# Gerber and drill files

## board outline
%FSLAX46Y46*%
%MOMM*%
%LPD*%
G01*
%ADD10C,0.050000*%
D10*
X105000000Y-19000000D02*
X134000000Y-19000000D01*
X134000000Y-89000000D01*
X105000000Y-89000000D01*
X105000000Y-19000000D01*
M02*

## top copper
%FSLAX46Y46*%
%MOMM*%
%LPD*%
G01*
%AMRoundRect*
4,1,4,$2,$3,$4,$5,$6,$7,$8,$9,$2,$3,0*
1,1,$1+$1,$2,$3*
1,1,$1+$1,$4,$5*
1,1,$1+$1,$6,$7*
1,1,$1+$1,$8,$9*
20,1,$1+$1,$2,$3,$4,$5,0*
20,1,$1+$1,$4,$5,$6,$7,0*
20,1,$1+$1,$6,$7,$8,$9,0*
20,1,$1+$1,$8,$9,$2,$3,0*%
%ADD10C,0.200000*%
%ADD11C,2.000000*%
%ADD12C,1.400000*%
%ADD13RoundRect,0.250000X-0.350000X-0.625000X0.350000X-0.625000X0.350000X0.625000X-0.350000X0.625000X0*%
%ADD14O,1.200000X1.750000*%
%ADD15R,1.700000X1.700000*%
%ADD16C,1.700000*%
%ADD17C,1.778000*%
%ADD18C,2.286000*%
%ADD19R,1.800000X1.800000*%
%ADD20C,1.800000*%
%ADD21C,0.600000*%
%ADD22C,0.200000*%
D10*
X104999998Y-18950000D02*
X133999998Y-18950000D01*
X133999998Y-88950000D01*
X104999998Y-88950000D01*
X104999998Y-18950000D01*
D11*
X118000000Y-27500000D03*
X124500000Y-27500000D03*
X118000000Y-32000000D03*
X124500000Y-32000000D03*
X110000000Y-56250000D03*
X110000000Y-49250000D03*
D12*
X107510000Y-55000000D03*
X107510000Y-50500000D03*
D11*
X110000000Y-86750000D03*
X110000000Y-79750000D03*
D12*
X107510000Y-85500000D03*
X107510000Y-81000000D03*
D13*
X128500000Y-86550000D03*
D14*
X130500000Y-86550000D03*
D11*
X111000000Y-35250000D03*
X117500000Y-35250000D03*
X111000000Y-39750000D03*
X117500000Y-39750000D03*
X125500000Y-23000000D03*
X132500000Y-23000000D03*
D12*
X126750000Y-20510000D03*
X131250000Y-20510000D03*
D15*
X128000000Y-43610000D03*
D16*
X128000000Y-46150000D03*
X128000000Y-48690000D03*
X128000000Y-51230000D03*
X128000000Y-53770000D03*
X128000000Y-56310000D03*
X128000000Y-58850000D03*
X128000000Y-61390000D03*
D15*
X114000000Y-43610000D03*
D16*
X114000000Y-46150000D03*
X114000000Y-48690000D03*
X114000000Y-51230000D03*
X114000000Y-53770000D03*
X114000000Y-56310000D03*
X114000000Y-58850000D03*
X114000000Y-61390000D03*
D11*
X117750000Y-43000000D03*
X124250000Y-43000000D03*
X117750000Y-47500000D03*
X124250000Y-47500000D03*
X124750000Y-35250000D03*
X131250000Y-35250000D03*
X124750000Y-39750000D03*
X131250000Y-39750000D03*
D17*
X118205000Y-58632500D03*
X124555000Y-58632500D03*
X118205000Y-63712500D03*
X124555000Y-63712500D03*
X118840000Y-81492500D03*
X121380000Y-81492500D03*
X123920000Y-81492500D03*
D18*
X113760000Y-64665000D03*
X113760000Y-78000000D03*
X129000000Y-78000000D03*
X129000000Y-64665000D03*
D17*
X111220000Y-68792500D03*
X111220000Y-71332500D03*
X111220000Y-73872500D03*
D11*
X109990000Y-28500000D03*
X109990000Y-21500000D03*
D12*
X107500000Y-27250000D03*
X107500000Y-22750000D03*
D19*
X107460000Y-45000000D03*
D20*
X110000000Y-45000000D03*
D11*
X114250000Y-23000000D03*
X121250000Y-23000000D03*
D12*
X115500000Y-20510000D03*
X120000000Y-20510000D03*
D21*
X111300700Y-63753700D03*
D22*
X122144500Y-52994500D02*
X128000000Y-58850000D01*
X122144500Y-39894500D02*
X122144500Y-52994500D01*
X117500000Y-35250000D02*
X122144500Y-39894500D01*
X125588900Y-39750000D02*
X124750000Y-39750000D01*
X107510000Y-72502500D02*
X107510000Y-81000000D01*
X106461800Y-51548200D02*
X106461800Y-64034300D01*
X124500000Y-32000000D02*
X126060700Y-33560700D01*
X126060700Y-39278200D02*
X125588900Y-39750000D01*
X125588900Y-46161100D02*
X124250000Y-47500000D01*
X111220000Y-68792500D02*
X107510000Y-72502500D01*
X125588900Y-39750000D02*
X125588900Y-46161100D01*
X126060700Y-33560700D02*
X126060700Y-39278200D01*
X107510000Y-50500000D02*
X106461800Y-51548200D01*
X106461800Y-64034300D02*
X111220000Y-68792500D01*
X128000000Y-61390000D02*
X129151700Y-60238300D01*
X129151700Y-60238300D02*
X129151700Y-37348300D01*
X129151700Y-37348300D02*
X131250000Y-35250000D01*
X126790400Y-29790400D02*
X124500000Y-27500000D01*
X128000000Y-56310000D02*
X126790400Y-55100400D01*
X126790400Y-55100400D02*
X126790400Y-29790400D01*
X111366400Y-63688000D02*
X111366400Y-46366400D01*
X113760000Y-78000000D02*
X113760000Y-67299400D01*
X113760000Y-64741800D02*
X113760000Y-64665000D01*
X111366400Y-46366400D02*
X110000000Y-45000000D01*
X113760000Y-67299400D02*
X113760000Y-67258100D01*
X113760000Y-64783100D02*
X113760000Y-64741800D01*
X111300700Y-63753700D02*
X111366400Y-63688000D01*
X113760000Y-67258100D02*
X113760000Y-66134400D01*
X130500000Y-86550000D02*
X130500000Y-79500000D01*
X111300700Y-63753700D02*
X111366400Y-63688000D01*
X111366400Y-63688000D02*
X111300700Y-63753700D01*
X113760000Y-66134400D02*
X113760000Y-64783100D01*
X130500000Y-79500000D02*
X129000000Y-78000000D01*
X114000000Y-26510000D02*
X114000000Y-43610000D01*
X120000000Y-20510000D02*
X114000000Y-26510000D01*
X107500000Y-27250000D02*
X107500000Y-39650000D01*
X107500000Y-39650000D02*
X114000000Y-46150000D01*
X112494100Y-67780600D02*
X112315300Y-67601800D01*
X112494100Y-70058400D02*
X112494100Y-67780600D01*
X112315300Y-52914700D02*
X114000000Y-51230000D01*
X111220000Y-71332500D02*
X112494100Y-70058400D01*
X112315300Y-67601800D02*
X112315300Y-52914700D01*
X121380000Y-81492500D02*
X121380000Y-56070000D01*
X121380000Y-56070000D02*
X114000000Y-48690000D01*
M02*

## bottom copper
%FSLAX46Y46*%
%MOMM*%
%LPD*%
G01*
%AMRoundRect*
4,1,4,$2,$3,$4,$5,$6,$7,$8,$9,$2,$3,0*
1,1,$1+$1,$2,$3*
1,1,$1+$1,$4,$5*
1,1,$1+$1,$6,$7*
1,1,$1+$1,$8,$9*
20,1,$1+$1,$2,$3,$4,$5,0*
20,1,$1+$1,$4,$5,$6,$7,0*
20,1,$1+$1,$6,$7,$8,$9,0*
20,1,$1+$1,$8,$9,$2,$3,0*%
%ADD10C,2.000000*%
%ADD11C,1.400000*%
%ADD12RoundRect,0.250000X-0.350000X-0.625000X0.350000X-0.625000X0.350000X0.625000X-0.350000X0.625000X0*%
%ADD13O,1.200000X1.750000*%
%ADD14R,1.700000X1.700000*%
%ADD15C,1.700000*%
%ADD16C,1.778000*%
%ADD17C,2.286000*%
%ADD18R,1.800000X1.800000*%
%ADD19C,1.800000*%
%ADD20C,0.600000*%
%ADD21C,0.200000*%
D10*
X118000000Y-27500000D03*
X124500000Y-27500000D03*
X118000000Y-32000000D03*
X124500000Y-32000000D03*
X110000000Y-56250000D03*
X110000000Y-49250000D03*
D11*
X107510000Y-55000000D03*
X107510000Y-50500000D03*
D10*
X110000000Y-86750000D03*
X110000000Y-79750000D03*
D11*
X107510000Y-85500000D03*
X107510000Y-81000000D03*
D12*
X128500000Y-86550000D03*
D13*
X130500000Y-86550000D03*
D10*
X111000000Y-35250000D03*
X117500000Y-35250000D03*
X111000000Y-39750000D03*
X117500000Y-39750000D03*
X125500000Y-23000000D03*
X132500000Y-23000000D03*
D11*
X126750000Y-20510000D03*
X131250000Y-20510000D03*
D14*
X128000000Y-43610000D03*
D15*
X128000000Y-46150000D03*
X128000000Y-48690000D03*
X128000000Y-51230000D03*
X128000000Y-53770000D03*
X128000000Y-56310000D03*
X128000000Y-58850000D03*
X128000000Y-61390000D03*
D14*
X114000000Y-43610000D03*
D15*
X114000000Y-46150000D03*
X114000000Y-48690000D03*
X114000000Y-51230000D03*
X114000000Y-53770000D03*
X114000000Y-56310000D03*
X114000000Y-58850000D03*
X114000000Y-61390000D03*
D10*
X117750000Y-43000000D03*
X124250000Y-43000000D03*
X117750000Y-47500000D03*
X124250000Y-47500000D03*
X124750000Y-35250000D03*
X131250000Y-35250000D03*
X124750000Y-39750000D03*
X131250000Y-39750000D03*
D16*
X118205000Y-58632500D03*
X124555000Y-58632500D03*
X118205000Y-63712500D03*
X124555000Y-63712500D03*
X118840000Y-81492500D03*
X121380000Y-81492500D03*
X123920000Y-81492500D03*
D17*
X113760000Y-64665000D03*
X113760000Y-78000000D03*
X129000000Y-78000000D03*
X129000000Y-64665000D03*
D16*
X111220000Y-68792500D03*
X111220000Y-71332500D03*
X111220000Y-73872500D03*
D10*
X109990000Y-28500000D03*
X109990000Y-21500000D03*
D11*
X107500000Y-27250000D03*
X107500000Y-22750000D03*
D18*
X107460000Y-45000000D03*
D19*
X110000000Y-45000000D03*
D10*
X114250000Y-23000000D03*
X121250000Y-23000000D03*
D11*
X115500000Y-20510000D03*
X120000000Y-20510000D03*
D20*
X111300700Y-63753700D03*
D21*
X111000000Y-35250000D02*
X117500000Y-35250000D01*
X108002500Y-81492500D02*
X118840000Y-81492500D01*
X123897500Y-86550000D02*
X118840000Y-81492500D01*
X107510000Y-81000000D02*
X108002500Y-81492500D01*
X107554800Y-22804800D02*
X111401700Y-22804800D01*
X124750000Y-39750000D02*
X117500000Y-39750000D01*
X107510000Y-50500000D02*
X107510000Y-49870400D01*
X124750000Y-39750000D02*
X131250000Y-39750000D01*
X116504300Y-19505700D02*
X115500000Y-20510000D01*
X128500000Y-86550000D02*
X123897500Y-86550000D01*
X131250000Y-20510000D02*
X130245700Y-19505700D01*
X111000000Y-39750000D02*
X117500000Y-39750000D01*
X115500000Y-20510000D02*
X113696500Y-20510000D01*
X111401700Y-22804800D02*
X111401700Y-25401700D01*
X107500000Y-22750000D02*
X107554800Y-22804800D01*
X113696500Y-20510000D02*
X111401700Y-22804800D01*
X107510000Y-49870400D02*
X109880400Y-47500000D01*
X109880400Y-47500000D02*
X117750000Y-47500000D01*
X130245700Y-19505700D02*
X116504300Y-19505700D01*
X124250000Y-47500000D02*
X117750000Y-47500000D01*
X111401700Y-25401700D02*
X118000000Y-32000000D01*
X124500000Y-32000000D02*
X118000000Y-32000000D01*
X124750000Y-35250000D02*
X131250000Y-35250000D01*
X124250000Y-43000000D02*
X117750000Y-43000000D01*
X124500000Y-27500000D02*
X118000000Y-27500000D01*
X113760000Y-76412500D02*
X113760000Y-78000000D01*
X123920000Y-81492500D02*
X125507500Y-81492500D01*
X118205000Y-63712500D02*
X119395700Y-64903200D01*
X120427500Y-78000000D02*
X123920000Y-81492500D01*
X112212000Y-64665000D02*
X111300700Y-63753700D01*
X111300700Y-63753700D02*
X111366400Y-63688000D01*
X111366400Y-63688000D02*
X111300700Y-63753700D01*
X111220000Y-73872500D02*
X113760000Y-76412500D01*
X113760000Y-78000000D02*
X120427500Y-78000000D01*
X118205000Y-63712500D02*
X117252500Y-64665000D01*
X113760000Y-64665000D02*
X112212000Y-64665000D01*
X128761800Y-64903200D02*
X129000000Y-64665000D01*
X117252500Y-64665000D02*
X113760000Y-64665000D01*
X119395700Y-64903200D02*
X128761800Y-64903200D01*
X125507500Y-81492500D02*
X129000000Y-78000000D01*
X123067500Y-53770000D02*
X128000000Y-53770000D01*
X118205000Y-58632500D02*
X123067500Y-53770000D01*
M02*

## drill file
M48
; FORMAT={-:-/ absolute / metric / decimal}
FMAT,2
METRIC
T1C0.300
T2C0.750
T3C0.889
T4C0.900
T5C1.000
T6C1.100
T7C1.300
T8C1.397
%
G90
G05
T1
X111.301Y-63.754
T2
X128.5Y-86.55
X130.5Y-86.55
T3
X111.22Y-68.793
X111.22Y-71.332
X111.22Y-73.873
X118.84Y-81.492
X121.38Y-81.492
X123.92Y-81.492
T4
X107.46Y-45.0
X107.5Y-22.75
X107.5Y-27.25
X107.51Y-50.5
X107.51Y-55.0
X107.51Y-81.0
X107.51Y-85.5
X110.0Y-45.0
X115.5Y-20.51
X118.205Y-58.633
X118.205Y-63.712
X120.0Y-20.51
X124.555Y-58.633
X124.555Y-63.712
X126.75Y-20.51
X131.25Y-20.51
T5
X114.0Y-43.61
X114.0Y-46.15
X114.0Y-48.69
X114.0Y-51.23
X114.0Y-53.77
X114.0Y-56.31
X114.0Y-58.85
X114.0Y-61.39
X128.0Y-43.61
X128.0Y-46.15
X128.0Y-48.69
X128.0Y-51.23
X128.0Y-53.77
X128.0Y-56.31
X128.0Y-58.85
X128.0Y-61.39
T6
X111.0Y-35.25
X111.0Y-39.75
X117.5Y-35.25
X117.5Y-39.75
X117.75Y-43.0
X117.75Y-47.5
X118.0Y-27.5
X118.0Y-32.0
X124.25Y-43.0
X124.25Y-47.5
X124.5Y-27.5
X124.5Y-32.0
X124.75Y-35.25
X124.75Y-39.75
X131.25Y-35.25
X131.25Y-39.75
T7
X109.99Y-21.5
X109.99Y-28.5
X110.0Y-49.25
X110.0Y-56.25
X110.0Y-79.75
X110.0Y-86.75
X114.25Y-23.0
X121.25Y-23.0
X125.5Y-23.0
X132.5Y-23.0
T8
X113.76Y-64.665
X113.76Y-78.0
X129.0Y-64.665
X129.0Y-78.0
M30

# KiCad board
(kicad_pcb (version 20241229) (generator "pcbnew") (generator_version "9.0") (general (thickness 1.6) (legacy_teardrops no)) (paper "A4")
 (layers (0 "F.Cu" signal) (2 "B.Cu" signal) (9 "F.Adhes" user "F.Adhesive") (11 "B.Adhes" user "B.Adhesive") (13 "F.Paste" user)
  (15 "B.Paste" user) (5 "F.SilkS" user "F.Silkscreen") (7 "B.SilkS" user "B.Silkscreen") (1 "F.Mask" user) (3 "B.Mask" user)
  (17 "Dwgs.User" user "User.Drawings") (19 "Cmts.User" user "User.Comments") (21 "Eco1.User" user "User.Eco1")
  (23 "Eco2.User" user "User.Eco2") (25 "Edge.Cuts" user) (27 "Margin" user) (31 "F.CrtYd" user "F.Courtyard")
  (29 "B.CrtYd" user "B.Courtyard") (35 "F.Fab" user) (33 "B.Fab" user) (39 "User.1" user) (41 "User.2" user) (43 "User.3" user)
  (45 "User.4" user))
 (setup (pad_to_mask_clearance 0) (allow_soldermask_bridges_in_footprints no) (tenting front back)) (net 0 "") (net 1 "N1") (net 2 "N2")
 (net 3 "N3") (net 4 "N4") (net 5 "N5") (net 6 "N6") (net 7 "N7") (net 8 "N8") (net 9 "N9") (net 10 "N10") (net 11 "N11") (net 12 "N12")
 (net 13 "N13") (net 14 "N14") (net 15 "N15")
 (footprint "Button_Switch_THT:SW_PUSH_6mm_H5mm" (layer "F.Cu") (at 118 27.5)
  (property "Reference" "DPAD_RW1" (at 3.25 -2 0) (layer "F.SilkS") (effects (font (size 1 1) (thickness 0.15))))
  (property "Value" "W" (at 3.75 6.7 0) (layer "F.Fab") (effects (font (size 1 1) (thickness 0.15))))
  (pad "1" thru_hole circle (at 0 0 90) (size 2 2) (drill 1.1) (layers "*.Cu" "*.Mask") (remove_unused_layers no) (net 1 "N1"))
  (pad "1" thru_hole circle (at 6.5 0 90) (size 2 2) (drill 1.1) (layers "*.Cu" "*.Mask") (remove_unused_layers no) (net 1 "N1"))
  (pad "2" thru_hole circle (at 0 4.5 90) (size 2 2) (drill 1.1) (layers "*.Cu" "*.Mask") (remove_unused_layers no) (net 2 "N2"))
  (pad "2" thru_hole circle (at 6.5 4.5 90) (size 2 2) (drill 1.1) (layers "*.Cu" "*.Mask") (remove_unused_layers no) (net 2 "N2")))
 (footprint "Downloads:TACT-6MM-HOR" (layer "F.Cu") (at 107.51 52.75 90)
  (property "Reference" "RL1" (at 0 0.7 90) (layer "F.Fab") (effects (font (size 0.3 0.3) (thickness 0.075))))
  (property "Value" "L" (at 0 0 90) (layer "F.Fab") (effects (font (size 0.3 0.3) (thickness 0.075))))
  (pad "" thru_hole circle (at -3.5 2.49 90) (size 2 2) (drill 1.3) (layers "*.Cu" "*.Mask" "F.SilkS") (remove_unused_layers no))
  (pad "" thru_hole circle (at 3.5 2.49 90) (size 2 2) (drill 1.3) (layers "*.Cu" "*.Mask" "F.SilkS") (remove_unused_layers no))
  (pad "1" thru_hole circle (at -2.25 0 90) (size 1.4 1.4) (drill 0.9) (layers "*.Cu" "*.Mask" "F.SilkS") (remove_unused_layers no)
   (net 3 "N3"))
  (pad "2" thru_hole circle (at 2.25 0 90) (size 1.4 1.4) (drill 0.9) (layers "*.Cu" "*.Mask" "F.SilkS") (remove_unused_layers no)
   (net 2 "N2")))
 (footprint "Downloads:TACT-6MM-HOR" (layer "F.Cu") (at 107.51 83.25 90)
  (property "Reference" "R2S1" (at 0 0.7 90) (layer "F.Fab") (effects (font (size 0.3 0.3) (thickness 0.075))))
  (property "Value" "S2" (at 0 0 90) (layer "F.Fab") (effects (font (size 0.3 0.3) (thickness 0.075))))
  (pad "" thru_hole circle (at -3.5 2.49 90) (size 2 2) (drill 1.3) (layers "*.Cu" "*.Mask" "F.SilkS") (remove_unused_layers no))
  (pad "" thru_hole circle (at 3.5 2.49 90) (size 2 2) (drill 1.3) (layers "*.Cu" "*.Mask" "F.SilkS") (remove_unused_layers no))
  (pad "1" thru_hole circle (at -2.25 0 90) (size 1.4 1.4) (drill 0.9) (layers "*.Cu" "*.Mask" "F.SilkS") (remove_unused_layers no)
   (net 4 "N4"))
  (pad "2" thru_hole circle (at 2.25 0 90) (size 1.4 1.4) (drill 0.9) (layers "*.Cu" "*.Mask" "F.SilkS") (remove_unused_layers no)
   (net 2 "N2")))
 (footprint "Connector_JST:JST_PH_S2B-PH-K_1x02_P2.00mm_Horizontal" (layer "F.Cu") (at 128.5 86.55)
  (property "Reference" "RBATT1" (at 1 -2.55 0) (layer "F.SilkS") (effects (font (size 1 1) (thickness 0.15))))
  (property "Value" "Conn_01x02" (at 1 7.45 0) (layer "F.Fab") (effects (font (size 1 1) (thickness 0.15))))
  (pad "1" thru_hole roundrect (at 0 0) (size 1.2 1.75) (drill 0.75) (layers "*.Cu" "*.Mask") (remove_unused_layers no)
   (roundrect_rratio 0.208333) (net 2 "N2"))
  (pad "2" thru_hole oval (at 2 0) (size 1.2 1.75) (drill 0.75) (layers "*.Cu" "*.Mask") (remove_unused_layers no) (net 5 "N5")))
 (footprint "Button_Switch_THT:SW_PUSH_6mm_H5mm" (layer "F.Cu") (at 111 35.25)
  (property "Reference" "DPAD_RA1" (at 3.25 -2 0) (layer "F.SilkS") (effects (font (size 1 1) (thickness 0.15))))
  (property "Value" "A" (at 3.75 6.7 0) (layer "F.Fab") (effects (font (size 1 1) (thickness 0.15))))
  (pad "1" thru_hole circle (at 0 0 90) (size 2 2) (drill 1.1) (layers "*.Cu" "*.Mask") (remove_unused_layers no) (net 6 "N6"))
  (pad "1" thru_hole circle (at 6.5 0 90) (size 2 2) (drill 1.1) (layers "*.Cu" "*.Mask") (remove_unused_layers no) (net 6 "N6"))
  (pad "2" thru_hole circle (at 0 4.5 90) (size 2 2) (drill 1.1) (layers "*.Cu" "*.Mask") (remove_unused_layers no) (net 2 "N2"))
  (pad "2" thru_hole circle (at 6.5 4.5 90) (size 2 2) (drill 1.1) (layers "*.Cu" "*.Mask") (remove_unused_layers no) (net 2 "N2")))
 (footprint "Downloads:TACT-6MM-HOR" (layer "F.Cu") (at 129 20.51)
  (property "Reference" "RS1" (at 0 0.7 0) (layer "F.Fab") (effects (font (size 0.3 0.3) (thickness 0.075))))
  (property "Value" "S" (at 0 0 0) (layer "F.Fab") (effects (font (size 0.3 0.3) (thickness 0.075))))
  (pad "" thru_hole circle (at -3.5 2.49) (size 2 2) (drill 1.3) (layers "*.Cu" "*.Mask" "F.SilkS") (remove_unused_layers no))
  (pad "" thru_hole circle (at 3.5 2.49) (size 2 2) (drill 1.3) (layers "*.Cu" "*.Mask" "F.SilkS") (remove_unused_layers no))
  (pad "1" thru_hole circle (at -2.25 0) (size 1.4 1.4) (drill 0.9) (layers "*.Cu" "*.Mask" "F.SilkS") (remove_unused_layers no)
   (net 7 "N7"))
  (pad "2" thru_hole circle (at 2.25 0) (size 1.4 1.4) (drill 0.9) (layers "*.Cu" "*.Mask" "F.SilkS") (remove_unused_layers no) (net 2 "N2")))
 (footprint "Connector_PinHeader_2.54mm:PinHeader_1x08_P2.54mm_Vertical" (layer "F.Cu") (at 128 43.61)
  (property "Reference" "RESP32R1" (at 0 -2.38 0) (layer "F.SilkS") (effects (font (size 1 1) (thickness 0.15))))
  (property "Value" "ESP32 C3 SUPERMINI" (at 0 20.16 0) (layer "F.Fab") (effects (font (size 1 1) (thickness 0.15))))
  (pad "1" thru_hole rect (at 0 0) (size 1.7 1.7) (drill 1) (layers "*.Cu" "*.Mask") (remove_unused_layers no))
  (pad "2" thru_hole circle (at 0 2.54) (size 1.7 1.7) (drill 1) (layers "*.Cu" "*.Mask") (remove_unused_layers no))
  (pad "3" thru_hole circle (at 0 5.08) (size 1.7 1.7) (drill 1) (layers "*.Cu" "*.Mask") (remove_unused_layers no))
  (pad "4" thru_hole circle (at 0 7.62) (size 1.7 1.7) (drill 1) (layers "*.Cu" "*.Mask") (remove_unused_layers no))
  (pad "5" thru_hole circle (at 0 10.16) (size 1.7 1.7) (drill 1) (layers "*.Cu" "*.Mask") (remove_unused_layers no) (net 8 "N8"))
  (pad "6" thru_hole circle (at 0 12.7) (size 1.7 1.7) (drill 1) (layers "*.Cu" "*.Mask") (remove_unused_layers no) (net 1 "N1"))
  (pad "7" thru_hole circle (at 0 15.24) (size 1.7 1.7) (drill 1) (layers "*.Cu" "*.Mask") (remove_unused_layers no) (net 6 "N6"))
  (pad "8" thru_hole circle (at 0 17.78) (size 1.7 1.7) (drill 1) (layers "*.Cu" "*.Mask") (remove_unused_layers no) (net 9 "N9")))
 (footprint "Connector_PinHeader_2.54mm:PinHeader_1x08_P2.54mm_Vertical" (layer "F.Cu") (at 114 43.61)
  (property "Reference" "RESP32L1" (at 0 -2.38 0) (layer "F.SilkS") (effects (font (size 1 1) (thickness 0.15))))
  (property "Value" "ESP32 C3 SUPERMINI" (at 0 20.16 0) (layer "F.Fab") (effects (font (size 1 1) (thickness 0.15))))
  (pad "1" thru_hole rect (at 0 0) (size 1.7 1.7) (drill 1) (layers "*.Cu" "*.Mask") (remove_unused_layers no) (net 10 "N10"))
  (pad "2" thru_hole circle (at 0 2.54) (size 1.7 1.7) (drill 1) (layers "*.Cu" "*.Mask") (remove_unused_layers no) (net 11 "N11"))
  (pad "3" thru_hole circle (at 0 5.08) (size 1.7 1.7) (drill 1) (layers "*.Cu" "*.Mask") (remove_unused_layers no) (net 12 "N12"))
  (pad "4" thru_hole circle (at 0 7.62) (size 1.7 1.7) (drill 1) (layers "*.Cu" "*.Mask") (remove_unused_layers no) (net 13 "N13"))
  (pad "5" thru_hole circle (at 0 10.16) (size 1.7 1.7) (drill 1) (layers "*.Cu" "*.Mask") (remove_unused_layers no))
  (pad "6" thru_hole circle (at 0 12.7) (size 1.7 1.7) (drill 1) (layers "*.Cu" "*.Mask") (remove_unused_layers no))
  (pad "7" thru_hole circle (at 0 15.24) (size 1.7 1.7) (drill 1) (layers "*.Cu" "*.Mask") (remove_unused_layers no))
  (pad "8" thru_hole circle (at 0 17.78) (size 1.7 1.7) (drill 1) (layers "*.Cu" "*.Mask") (remove_unused_layers no)))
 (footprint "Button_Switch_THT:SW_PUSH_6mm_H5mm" (layer "F.Cu") (at 117.75 43)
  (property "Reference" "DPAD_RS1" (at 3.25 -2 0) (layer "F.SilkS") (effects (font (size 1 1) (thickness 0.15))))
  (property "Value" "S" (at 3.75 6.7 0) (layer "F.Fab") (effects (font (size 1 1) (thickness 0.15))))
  (pad "1" thru_hole circle (at 0 0 90) (size 2 2) (drill 1.1) (layers "*.Cu" "*.Mask") (remove_unused_layers no) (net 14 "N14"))
  (pad "1" thru_hole circle (at 6.5 0 90) (size 2 2) (drill 1.1) (layers "*.Cu" "*.Mask") (remove_unused_layers no) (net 14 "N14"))
  (pad "2" thru_hole circle (at 0 4.5 90) (size 2 2) (drill 1.1) (layers "*.Cu" "*.Mask") (remove_unused_layers no) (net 2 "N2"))
  (pad "2" thru_hole circle (at 6.5 4.5 90) (size 2 2) (drill 1.1) (layers "*.Cu" "*.Mask") (remove_unused_layers no) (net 2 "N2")))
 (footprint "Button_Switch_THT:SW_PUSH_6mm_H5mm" (layer "F.Cu") (at 124.75 35.25)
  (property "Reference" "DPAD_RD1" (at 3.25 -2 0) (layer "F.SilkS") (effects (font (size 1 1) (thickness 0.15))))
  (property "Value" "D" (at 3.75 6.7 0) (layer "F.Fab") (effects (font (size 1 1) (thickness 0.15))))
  (pad "1" thru_hole circle (at 0 0 90) (size 2 2) (drill 1.1) (layers "*.Cu" "*.Mask") (remove_unused_layers no) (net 9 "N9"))
  (pad "1" thru_hole circle (at 6.5 0 90) (size 2 2) (drill 1.1) (layers "*.Cu" "*.Mask") (remove_unused_layers no) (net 9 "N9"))
  (pad "2" thru_hole circle (at 0 4.5 90) (size 2 2) (drill 1.1) (layers "*.Cu" "*.Mask") (remove_unused_layers no) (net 2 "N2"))
  (pad "2" thru_hole circle (at 6.5 4.5 90) (size 2 2) (drill 1.1) (layers "*.Cu" "*.Mask") (remove_unused_layers no) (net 2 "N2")))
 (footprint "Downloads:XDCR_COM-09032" (layer "F.Cu") (at 121.38 71.3325)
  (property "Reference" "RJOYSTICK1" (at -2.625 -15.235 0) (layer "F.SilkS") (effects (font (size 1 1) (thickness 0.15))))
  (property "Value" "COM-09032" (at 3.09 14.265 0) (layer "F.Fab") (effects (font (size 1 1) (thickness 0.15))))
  (pad "B1A" thru_hole circle (at -3.175 -12.7) (size 1.778 1.778) (drill 0.9) (layers "*.Cu" "*.Mask") (remove_unused_layers no)
   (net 8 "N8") (solder_mask_margin 0.102))
  (pad "B1B" thru_hole circle (at 3.175 -12.7) (size 1.778 1.778) (drill 0.9) (layers "*.Cu" "*.Mask") (remove_unused_layers no)
   (solder_mask_margin 0.102))
  (pad "B2A" thru_hole circle (at -3.175 -7.62) (size 1.778 1.778) (drill 0.9) (layers "*.Cu" "*.Mask") (remove_unused_layers no)
   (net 5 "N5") (solder_mask_margin 0.102))
  (pad "B2B" thru_hole circle (at 3.175 -7.62) (size 1.778 1.778) (drill 0.9) (layers "*.Cu" "*.Mask") (remove_unused_layers no)
   (solder_mask_margin 0.102))
  (pad "H1" thru_hole circle (at -2.54 10.16) (size 1.778 1.778) (drill 0.889) (layers "*.Cu" "*.Mask") (remove_unused_layers no)
   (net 2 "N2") (solder_mask_margin 0.102))
  (pad "H2" thru_hole circle (at 0 10.16) (size 1.778 1.778) (drill 0.889) (layers "*.Cu" "*.Mask") (remove_unused_layers no) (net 12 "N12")
   (solder_mask_margin 0.102))
  (pad "H3" thru_hole circle (at 2.54 10.16) (size 1.778 1.778) (drill 0.889) (layers "*.Cu" "*.Mask") (remove_unused_layers no)
   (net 5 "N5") (solder_mask_margin 0.102))
  (pad "S1" thru_hole circle (at -7.62 -6.6675) (size 2.286 2.286) (drill 1.397) (layers "*.Cu" "*.Mask") (remove_unused_layers no)
   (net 5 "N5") (solder_mask_margin 0.102))
  (pad "S2" thru_hole circle (at -7.62 6.6675) (size 2.286 2.286) (drill 1.397) (layers "*.Cu" "*.Mask") (remove_unused_layers no)
   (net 5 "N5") (solder_mask_margin 0.102))
  (pad "S3" thru_hole circle (at 7.62 6.6675) (size 2.286 2.286) (drill 1.397) (layers "*.Cu" "*.Mask") (remove_unused_layers no)
   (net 5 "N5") (solder_mask_margin 0.102))
  (pad "S4" thru_hole circle (at 7.62 -6.6675) (size 2.286 2.286) (drill 1.397) (layers "*.Cu" "*.Mask") (remove_unused_layers no)
   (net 5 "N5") (solder_mask_margin 0.102))
  (pad "V1" thru_hole circle (at -10.16 -2.54) (size 1.778 1.778) (drill 0.889) (layers "*.Cu" "*.Mask") (remove_unused_layers no)
   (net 2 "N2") (solder_mask_margin 0.102))
  (pad "V2" thru_hole circle (at -10.16 0) (size 1.778 1.778) (drill 0.889) (layers "*.Cu" "*.Mask") (remove_unused_layers no)
   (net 13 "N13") (solder_mask_margin 0.102))
  (pad "V3" thru_hole circle (at -10.16 2.54) (size 1.778 1.778) (drill 0.889) (layers "*.Cu" "*.Mask") (remove_unused_layers no)
   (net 5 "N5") (solder_mask_margin 0.102)))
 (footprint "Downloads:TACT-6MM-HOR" (layer "F.Cu") (at 107.5 25 90)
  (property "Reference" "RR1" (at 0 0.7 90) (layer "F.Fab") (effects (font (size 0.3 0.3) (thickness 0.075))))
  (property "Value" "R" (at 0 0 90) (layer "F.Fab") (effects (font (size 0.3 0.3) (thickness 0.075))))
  (pad "" thru_hole circle (at -3.5 2.49 90) (size 2 2) (drill 1.3) (layers "*.Cu" "*.Mask" "F.SilkS") (remove_unused_layers no))
  (pad "" thru_hole circle (at 3.5 2.49 90) (size 2 2) (drill 1.3) (layers "*.Cu" "*.Mask" "F.SilkS") (remove_unused_layers no))
  (pad "1" thru_hole circle (at -2.25 0 90) (size 1.4 1.4) (drill 0.9) (layers "*.Cu" "*.Mask" "F.SilkS") (remove_unused_layers no)
   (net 11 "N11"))
  (pad "2" thru_hole circle (at 2.25 0 90) (size 1.4 1.4) (drill 0.9) (layers "*.Cu" "*.Mask" "F.SilkS") (remove_unused_layers no)
   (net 2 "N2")))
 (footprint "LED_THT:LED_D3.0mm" (layer "F.Cu") (at 107.46 45)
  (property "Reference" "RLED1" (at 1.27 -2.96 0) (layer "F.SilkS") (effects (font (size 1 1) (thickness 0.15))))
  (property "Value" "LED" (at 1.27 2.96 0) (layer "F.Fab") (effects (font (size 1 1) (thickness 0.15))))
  (pad "1" thru_hole rect (at 0 0) (size 1.8 1.8) (drill 0.9) (layers "*.Cu" "*.Mask") (remove_unused_layers no) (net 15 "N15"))
  (pad "2" thru_hole circle (at 2.54 0) (size 1.8 1.8) (drill 0.9) (layers "*.Cu" "*.Mask") (remove_unused_layers no) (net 5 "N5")))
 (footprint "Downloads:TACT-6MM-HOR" (layer "F.Cu") (at 117.75 20.51)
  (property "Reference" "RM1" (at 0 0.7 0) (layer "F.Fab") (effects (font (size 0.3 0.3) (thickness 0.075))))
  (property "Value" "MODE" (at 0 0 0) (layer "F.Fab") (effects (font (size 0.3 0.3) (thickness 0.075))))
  (pad "" thru_hole circle (at -3.5 2.49) (size 2 2) (drill 1.3) (layers "*.Cu" "*.Mask" "F.SilkS") (remove_unused_layers no))
  (pad "" thru_hole circle (at 3.5 2.49) (size 2 2) (drill 1.3) (layers "*.Cu" "*.Mask" "F.SilkS") (remove_unused_layers no))
  (pad "1" thru_hole circle (at -2.25 0) (size 1.4 1.4) (drill 0.9) (layers "*.Cu" "*.Mask" "F.SilkS") (remove_unused_layers no)
   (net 2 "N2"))
  (pad "2" thru_hole circle (at 2.25 0) (size 1.4 1.4) (drill 0.9) (layers "*.Cu" "*.Mask" "F.SilkS") (remove_unused_layers no)
   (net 10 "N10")))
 (gr_rect (start 104.999998 18.95) (end 133.999998 88.95) (stroke (width 0.2) (type default)) (fill no) (layer "F.Cu"))
 (gr_rect (start 105 19) (end 134 89) (stroke (width 0.05) (type default)) (fill no) (layer "Edge.Cuts"))
 (segment (start 122.1445 52.9945) (end 128 58.85) (width 0.2) (layer "F.Cu") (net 6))
 (segment (start 122.1445 39.8945) (end 122.1445 52.9945) (width 0.2) (layer "F.Cu") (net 6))
 (segment (start 117.5 35.25) (end 122.1445 39.8945) (width 0.2) (layer "F.Cu") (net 6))
 (segment (start 111 35.25) (end 117.5 35.25) (width 0.2) (layer "B.Cu") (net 6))
 (segment (start 125.5889 39.75) (end 124.75 39.75) (width 0.2) (layer "F.Cu") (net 2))
 (segment (start 107.51 72.5025) (end 107.51 81) (width 0.2) (layer "F.Cu") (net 2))
 (segment (start 106.4618 51.5482) (end 106.4618 64.0343) (width 0.2) (layer "F.Cu") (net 2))
 (segment (start 124.5 32) (end 126.0607 33.5607) (width 0.2) (layer "F.Cu") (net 2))
 (segment (start 126.0607 39.2782) (end 125.5889 39.75) (width 0.2) (layer "F.Cu") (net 2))
 (segment (start 125.5889 46.1611) (end 124.25 47.5) (width 0.2) (layer "F.Cu") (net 2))
 (segment (start 111.22 68.7925) (end 107.51 72.5025) (width 0.2) (layer "F.Cu") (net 2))
 (segment (start 125.5889 39.75) (end 125.5889 46.1611) (width 0.2) (layer "F.Cu") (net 2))
 (segment (start 126.0607 33.5607) (end 126.0607 39.2782) (width 0.2) (layer "F.Cu") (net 2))
 (segment (start 107.51 50.5) (end 106.4618 51.5482) (width 0.2) (layer "F.Cu") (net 2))
 (segment (start 106.4618 64.0343) (end 111.22 68.7925) (width 0.2) (layer "F.Cu") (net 2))
 (segment (start 108.0025 81.4925) (end 118.84 81.4925) (width 0.2) (layer "B.Cu") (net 2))
 (segment (start 123.8975 86.55) (end 118.84 81.4925) (width 0.2) (layer "B.Cu") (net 2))
 (segment (start 107.51 81) (end 108.0025 81.4925) (width 0.2) (layer "B.Cu") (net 2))
 (segment (start 107.5548 22.8048) (end 111.4017 22.8048) (width 0.2) (layer "B.Cu") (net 2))
 (segment (start 124.75 39.75) (end 117.5 39.75) (width 0.2) (layer "B.Cu") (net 2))
 (segment (start 107.51 50.5) (end 107.51 49.8704) (width 0.2) (layer "B.Cu") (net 2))
 (segment (start 124.75 39.75) (end 131.25 39.75) (width 0.2) (layer "B.Cu") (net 2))
 (segment (start 116.5043 19.5057) (end 115.5 20.51) (width 0.2) (layer "B.Cu") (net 2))
 (segment (start 128.5 86.55) (end 123.8975 86.55) (width 0.2) (layer "B.Cu") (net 2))
 (segment (start 131.25 20.51) (end 130.2457 19.5057) (width 0.2) (layer "B.Cu") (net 2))
 (segment (start 111 39.75) (end 117.5 39.75) (width 0.2) (layer "B.Cu") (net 2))
 (segment (start 115.5 20.51) (end 113.6965 20.51) (width 0.2) (layer "B.Cu") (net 2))
 (segment (start 111.4017 22.8048) (end 111.4017 25.4017) (width 0.2) (layer "B.Cu") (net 2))
 (segment (start 107.5 22.75) (end 107.5548 22.8048) (width 0.2) (layer "B.Cu") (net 2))
 (segment (start 113.6965 20.51) (end 111.4017 22.8048) (width 0.2) (layer "B.Cu") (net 2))
 (segment (start 107.51 49.8704) (end 109.8804 47.5) (width 0.2) (layer "B.Cu") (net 2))
 (segment (start 109.8804 47.5) (end 117.75 47.5) (width 0.2) (layer "B.Cu") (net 2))
 (segment (start 130.2457 19.5057) (end 116.5043 19.5057) (width 0.2) (layer "B.Cu") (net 2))
 (segment (start 124.25 47.5) (end 117.75 47.5) (width 0.2) (layer "B.Cu") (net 2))
 (segment (start 111.4017 25.4017) (end 118 32) (width 0.2) (layer "B.Cu") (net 2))
 (segment (start 124.5 32) (end 118 32) (width 0.2) (layer "B.Cu") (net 2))
 (segment (start 128 61.39) (end 129.1517 60.2383) (width 0.2) (layer "F.Cu") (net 9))
 (segment (start 129.1517 60.2383) (end 129.1517 37.3483) (width 0.2) (layer "F.Cu") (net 9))
 (segment (start 129.1517 37.3483) (end 131.25 35.25) (width 0.2) (layer "F.Cu") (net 9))
 (segment (start 124.75 35.25) (end 131.25 35.25) (width 0.2) (layer "B.Cu") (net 9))
 (segment (start 124.25 43) (end 117.75 43) (width 0.2) (layer "B.Cu") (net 14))
 (segment (start 126.7904 29.7904) (end 124.5 27.5) (width 0.2) (layer "F.Cu") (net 1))
 (segment (start 128 56.31) (end 126.7904 55.1004) (width 0.2) (layer "F.Cu") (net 1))
 (segment (start 126.7904 55.1004) (end 126.7904 29.7904) (width 0.2) (layer "F.Cu") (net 1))
 (segment (start 124.5 27.5) (end 118 27.5) (width 0.2) (layer "B.Cu") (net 1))
 (segment (start 111.3664 63.688) (end 111.3664 46.3664) (width 0.2) (layer "F.Cu") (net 5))
 (segment (start 113.76 78) (end 113.76 67.2994) (width 0.2) (layer "F.Cu") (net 5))
 (segment (start 113.76 64.7418) (end 113.76 64.665) (width 0.2) (layer "F.Cu") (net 5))
 (segment (start 111.3664 46.3664) (end 110 45) (width 0.2) (layer "F.Cu") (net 5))
 (segment (start 113.76 67.2994) (end 113.76 67.2581) (width 0.2) (layer "F.Cu") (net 5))
 (segment (start 113.76 64.7831) (end 113.76 64.7418) (width 0.2) (layer "F.Cu") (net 5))
 (segment (start 111.3007 63.7537) (end 111.3664 63.688) (width 0.2) (layer "F.Cu") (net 5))
 (segment (start 113.76 67.2581) (end 113.76 66.1344) (width 0.2) (layer "F.Cu") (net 5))
 (segment (start 130.5 86.55) (end 130.5 79.5) (width 0.2) (layer "F.Cu") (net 5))
 (segment (start 111.3007 63.7537) (end 111.3664 63.688) (width 0.2) (layer "F.Cu") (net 5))
 (segment (start 111.3664 63.688) (end 111.3007 63.7537) (width 0.2) (layer "F.Cu") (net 5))
 (segment (start 113.76 66.1344) (end 113.76 64.7831) (width 0.2) (layer "F.Cu") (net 5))
 (segment (start 130.5 79.5) (end 129 78) (width 0.2) (layer "F.Cu") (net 5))
 (via (at 111.3007 63.7537) (size 0.6) (drill 0.3) (layers "F.Cu" "B.Cu") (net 5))
 (segment (start 113.76 76.4125) (end 113.76 78) (width 0.2) (layer "B.Cu") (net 5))
 (segment (start 123.92 81.4925) (end 125.5075 81.4925) (width 0.2) (layer "B.Cu") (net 5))
 (segment (start 118.205 63.7125) (end 119.3957 64.9032) (width 0.2) (layer "B.Cu") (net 5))
 (segment (start 120.4275 78) (end 123.92 81.4925) (width 0.2) (layer "B.Cu") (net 5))
 (segment (start 112.212 64.665) (end 111.3007 63.7537) (width 0.2) (layer "B.Cu") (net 5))
 (segment (start 111.3007 63.7537) (end 111.3664 63.688) (width 0.2) (layer "B.Cu") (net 5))
 (segment (start 111.3664 63.688) (end 111.3007 63.7537) (width 0.2) (layer "B.Cu") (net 5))
 (segment (start 111.22 73.8725) (end 113.76 76.4125) (width 0.2) (layer "B.Cu") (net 5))
 (segment (start 113.76 78) (end 120.4275 78) (width 0.2) (layer "B.Cu") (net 5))
 (segment (start 118.205 63.7125) (end 117.2525 64.665) (width 0.2) (layer "B.Cu") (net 5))
 (segment (start 113.76 64.665) (end 112.212 64.665) (width 0.2) (layer "B.Cu") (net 5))
 (segment (start 128.7618 64.9032) (end 129 64.665) (width 0.2) (layer "B.Cu") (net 5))
 (segment (start 117.2525 64.665) (end 113.76 64.665) (width 0.2) (layer "B.Cu") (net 5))
 (segment (start 119.3957 64.9032) (end 128.7618 64.9032) (width 0.2) (layer "B.Cu") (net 5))
 (segment (start 125.5075 81.4925) (end 129 78) (width 0.2) (layer "B.Cu") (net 5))
 (segment (start 114 26.51) (end 114 43.61) (width 0.2) (layer "F.Cu") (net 10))
 (segment (start 120 20.51) (end 114 26.51) (width 0.2) (layer "F.Cu") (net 10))
 (segment (start 107.5 27.25) (end 107.5 39.65) (width 0.2) (layer "F.Cu") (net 11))
 (segment (start 107.5 39.65) (end 114 46.15) (width 0.2) (layer "F.Cu") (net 11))
 (segment (start 112.4941 67.7806) (end 112.3153 67.6018) (width 0.2) (layer "F.Cu") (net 13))
 (segment (start 112.4941 70.0584) (end 112.4941 67.7806) (width 0.2) (layer "F.Cu") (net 13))
 (segment (start 112.3153 52.9147) (end 114 51.23) (width 0.2) (layer "F.Cu") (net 13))
 (segment (start 111.22 71.3325) (end 112.4941 70.0584) (width 0.2) (layer "F.Cu") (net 13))
 (segment (start 112.3153 67.6018) (end 112.3153 52.9147) (width 0.2) (layer "F.Cu") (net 13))
 (segment (start 121.38 81.4925) (end 121.38 56.07) (width 0.2) (layer "F.Cu") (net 12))
 (segment (start 121.38 56.07) (end 114 48.69) (width 0.2) (layer "F.Cu") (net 12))
 (segment (start 123.0675 53.77) (end 128 53.77) (width 0.2) (layer "B.Cu") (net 8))
 (segment (start 118.205 58.6325) (end 123.0675 53.77) (width 0.2) (layer "B.Cu") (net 8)))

